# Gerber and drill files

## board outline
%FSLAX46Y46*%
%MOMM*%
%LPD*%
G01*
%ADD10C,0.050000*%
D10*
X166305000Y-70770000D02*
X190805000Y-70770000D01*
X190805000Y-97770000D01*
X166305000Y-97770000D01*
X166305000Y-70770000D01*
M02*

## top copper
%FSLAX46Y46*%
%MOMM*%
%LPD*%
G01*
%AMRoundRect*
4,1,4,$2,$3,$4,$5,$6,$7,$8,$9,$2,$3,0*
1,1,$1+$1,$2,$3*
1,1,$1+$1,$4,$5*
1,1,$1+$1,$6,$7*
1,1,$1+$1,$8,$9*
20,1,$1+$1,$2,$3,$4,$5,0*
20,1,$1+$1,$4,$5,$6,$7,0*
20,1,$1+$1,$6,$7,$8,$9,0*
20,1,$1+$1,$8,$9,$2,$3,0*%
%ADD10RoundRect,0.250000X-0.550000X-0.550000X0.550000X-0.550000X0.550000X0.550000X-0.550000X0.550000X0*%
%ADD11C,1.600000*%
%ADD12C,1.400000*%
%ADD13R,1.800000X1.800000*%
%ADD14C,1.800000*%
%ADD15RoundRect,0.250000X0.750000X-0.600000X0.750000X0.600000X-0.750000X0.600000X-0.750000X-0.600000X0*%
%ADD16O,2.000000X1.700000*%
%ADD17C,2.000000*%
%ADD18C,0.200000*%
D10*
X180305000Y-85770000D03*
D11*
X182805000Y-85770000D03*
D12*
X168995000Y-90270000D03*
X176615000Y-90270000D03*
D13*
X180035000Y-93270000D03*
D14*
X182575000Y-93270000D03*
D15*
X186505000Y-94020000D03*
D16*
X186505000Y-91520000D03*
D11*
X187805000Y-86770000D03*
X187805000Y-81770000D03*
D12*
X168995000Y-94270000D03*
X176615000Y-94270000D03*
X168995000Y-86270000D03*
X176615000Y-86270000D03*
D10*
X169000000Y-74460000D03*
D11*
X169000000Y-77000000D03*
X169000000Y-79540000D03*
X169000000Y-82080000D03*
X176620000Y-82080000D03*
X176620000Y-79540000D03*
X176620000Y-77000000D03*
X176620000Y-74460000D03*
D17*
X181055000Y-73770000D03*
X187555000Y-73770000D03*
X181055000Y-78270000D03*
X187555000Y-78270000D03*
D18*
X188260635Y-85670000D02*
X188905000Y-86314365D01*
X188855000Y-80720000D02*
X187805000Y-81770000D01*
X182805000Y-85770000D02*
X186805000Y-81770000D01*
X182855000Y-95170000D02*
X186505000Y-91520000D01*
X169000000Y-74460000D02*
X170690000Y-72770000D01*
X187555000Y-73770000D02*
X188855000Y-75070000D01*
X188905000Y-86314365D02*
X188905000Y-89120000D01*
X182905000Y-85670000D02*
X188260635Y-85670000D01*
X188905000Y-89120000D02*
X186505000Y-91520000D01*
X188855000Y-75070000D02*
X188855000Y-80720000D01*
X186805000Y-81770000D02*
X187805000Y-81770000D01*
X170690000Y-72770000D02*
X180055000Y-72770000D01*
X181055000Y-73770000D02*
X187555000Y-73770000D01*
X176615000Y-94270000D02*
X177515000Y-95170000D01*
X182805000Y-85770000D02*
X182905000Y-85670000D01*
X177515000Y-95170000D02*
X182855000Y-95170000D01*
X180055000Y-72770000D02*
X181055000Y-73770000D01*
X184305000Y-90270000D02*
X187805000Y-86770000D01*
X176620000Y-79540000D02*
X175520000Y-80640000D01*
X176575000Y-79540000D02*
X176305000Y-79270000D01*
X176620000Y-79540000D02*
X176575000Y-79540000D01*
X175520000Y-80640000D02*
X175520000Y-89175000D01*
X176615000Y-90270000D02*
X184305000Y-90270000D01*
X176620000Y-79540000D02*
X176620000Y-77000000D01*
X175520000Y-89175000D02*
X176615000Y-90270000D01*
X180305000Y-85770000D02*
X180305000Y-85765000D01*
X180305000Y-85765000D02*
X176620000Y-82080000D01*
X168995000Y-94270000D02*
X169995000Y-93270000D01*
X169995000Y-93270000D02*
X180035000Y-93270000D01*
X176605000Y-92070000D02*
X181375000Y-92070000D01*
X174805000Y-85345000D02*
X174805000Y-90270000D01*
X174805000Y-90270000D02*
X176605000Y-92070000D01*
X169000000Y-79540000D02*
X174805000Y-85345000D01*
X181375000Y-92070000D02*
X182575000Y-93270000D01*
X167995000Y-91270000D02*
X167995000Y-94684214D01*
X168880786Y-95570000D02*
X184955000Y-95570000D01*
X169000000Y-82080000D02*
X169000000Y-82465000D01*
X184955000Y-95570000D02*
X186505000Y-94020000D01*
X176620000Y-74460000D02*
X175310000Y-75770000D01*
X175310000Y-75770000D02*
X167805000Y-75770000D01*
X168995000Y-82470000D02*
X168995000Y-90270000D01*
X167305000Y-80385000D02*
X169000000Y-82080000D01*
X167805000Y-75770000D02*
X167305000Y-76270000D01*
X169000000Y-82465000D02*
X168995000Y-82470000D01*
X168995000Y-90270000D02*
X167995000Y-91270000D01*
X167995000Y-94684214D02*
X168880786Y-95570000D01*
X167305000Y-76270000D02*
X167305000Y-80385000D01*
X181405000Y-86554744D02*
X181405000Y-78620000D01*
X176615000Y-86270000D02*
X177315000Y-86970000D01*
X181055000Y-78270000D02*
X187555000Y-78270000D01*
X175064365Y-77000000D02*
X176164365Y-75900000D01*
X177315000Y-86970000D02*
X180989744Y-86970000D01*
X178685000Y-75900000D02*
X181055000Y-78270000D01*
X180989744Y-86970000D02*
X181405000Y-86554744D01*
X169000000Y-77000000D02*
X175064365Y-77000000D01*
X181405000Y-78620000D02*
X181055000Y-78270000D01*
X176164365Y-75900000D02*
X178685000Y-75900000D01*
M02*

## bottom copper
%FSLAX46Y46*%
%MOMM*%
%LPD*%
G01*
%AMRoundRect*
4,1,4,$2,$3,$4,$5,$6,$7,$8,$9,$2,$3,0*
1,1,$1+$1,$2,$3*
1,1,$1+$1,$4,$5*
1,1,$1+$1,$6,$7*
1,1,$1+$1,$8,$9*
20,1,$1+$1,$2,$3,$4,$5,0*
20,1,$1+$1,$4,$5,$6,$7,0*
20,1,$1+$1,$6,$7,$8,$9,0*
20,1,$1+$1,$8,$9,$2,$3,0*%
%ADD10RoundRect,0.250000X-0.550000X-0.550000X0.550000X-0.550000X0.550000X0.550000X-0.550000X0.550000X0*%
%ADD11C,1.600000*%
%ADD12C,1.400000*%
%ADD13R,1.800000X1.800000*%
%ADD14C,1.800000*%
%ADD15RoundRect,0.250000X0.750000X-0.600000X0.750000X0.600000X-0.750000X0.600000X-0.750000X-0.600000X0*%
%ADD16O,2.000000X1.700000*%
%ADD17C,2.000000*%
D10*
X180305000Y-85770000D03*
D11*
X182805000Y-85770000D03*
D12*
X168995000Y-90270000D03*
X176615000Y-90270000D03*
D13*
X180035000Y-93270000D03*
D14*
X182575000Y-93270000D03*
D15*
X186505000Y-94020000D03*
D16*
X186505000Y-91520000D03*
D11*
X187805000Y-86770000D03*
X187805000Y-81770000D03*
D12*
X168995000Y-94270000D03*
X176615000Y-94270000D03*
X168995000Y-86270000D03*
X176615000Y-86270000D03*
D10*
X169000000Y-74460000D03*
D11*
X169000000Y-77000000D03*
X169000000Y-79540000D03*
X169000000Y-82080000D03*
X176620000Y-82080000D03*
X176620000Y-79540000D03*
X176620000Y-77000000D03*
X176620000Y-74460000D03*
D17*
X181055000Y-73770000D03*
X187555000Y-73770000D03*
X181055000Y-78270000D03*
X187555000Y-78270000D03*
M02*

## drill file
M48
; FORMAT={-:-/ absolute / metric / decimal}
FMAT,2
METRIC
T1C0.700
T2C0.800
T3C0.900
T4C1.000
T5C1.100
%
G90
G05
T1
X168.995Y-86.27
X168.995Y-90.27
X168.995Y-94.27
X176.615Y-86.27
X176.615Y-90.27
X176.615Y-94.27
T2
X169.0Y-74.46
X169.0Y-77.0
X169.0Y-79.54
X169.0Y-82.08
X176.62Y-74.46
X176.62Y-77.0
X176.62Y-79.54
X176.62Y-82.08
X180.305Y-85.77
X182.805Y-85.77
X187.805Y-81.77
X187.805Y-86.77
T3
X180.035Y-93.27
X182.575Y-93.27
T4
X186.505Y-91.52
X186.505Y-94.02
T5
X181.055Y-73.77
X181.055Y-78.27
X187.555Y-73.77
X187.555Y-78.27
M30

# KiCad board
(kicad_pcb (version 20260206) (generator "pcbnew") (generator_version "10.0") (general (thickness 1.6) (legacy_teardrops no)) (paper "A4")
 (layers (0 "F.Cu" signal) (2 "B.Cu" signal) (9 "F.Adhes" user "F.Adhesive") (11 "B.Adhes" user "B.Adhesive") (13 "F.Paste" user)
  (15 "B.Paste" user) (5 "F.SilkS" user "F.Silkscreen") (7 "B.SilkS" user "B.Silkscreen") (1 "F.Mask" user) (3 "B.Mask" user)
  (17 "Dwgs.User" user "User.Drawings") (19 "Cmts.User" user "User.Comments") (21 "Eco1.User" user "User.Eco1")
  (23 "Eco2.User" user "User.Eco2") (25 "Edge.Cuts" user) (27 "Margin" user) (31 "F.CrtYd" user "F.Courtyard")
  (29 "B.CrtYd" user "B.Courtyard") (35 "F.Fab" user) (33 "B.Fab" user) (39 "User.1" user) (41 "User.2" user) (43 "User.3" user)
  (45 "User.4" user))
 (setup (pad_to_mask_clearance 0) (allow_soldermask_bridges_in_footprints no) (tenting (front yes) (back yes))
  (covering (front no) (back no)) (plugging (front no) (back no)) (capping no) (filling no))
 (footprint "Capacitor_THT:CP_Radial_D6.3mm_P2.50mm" (layer "F.Cu") (at 180.305 85.77)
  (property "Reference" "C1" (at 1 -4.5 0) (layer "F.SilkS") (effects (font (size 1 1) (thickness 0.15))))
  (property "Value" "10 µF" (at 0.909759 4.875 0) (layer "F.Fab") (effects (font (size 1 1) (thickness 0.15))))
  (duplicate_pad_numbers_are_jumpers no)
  (pad "1" thru_hole roundrect (at 0 0) (size 1.6 1.6) (drill 0.8) (layers "*.Cu" "*.Mask") (remove_unused_layers no)
   (roundrect_rratio 0.15625) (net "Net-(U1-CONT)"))
  (pad "2" thru_hole circle (at 2.5 0) (size 1.6 1.6) (drill 0.8) (layers "*.Cu" "*.Mask") (remove_unused_layers no) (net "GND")))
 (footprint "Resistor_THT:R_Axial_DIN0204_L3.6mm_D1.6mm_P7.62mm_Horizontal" (layer "F.Cu") (at 168.995 90.27)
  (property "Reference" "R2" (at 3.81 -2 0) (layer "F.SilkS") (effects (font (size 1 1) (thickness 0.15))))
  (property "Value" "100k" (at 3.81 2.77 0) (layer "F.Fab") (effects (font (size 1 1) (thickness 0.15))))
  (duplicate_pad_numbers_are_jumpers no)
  (pad "1" thru_hole circle (at 0 0) (size 1.4 1.4) (drill 0.7) (layers "*.Cu" "*.Mask") (remove_unused_layers no) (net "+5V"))
  (pad "2" thru_hole circle (at 7.62 0) (size 1.4 1.4) (drill 0.7) (layers "*.Cu" "*.Mask") (remove_unused_layers no) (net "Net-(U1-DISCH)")))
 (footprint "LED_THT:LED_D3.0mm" (layer "F.Cu") (at 180.035 93.27)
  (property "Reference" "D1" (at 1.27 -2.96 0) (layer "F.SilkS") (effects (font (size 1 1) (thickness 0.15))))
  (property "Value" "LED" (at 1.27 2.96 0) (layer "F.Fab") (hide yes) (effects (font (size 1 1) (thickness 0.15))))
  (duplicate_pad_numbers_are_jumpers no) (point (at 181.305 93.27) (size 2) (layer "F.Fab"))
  (pad "1" thru_hole rect (at 0 0) (size 1.8 1.8) (drill 0.9) (layers "*.Cu" "*.Mask") (remove_unused_layers no) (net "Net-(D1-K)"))
  (pad "2" thru_hole circle (at 2.54 0) (size 1.8 1.8) (drill 0.9) (layers "*.Cu" "*.Mask") (remove_unused_layers no) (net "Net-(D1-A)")))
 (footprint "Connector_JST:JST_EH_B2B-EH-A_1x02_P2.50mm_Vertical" (layer "F.Cu") (at 186.505 94.02 90)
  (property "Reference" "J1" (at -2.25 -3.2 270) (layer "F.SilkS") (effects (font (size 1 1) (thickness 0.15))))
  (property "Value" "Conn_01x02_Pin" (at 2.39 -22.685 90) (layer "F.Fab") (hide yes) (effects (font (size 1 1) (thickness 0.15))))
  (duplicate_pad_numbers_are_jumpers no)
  (pad "1" thru_hole roundrect (at 0 0 90) (size 1.7 2) (drill 1) (layers "*.Cu" "*.Mask") (remove_unused_layers no)
   (roundrect_rratio 0.147059) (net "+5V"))
  (pad "2" thru_hole oval (at 2.5 0 90) (size 1.7 2) (drill 1) (layers "*.Cu" "*.Mask") (remove_unused_layers no) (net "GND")))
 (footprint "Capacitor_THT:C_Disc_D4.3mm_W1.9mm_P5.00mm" (layer "F.Cu") (at 187.805 86.77 90)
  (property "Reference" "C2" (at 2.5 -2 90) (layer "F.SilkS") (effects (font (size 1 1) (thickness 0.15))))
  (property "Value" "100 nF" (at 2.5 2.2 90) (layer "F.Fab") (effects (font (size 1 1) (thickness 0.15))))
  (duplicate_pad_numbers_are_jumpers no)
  (pad "1" thru_hole circle (at 0 0 90) (size 1.6 1.6) (drill 0.8) (layers "*.Cu" "*.Mask") (remove_unused_layers no) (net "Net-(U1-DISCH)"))
  (pad "2" thru_hole circle (at 5 0 90) (size 1.6 1.6) (drill 0.8) (layers "*.Cu" "*.Mask") (remove_unused_layers no) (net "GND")))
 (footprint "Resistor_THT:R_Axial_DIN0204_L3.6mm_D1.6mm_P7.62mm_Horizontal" (layer "F.Cu") (at 168.995 94.27)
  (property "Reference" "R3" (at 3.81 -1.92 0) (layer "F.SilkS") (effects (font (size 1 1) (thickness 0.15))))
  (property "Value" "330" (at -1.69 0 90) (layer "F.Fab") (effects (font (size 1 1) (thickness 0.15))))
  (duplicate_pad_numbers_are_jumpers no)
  (pad "1" thru_hole circle (at 0 0) (size 1.4 1.4) (drill 0.7) (layers "*.Cu" "*.Mask") (remove_unused_layers no) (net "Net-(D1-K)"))
  (pad "2" thru_hole circle (at 7.62 0) (size 1.4 1.4) (drill 0.7) (layers "*.Cu" "*.Mask") (remove_unused_layers no) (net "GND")))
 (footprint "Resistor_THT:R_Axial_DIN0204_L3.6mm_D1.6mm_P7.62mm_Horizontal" (layer "F.Cu") (at 168.995 86.27)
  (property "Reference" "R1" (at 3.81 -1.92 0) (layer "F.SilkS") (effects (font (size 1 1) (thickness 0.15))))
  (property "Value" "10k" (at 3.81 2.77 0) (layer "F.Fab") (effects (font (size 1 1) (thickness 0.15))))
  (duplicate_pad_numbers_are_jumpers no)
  (pad "1" thru_hole circle (at 0 0) (size 1.4 1.4) (drill 0.7) (layers "*.Cu" "*.Mask") (remove_unused_layers no) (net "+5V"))
  (pad "2" thru_hole circle (at 7.62 0) (size 1.4 1.4) (drill 0.7) (layers "*.Cu" "*.Mask") (remove_unused_layers no) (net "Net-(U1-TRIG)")))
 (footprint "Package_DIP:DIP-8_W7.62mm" (layer "F.Cu") (at 169 74.46)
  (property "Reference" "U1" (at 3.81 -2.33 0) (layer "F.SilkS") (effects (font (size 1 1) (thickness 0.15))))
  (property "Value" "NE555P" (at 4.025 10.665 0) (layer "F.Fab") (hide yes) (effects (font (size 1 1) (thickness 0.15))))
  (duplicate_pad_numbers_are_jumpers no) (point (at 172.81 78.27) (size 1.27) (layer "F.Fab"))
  (pad "1" thru_hole roundrect (at 0 0) (size 1.6 1.6) (drill 0.8) (layers "*.Cu" "*.Mask") (remove_unused_layers no)
   (roundrect_rratio 0.15625) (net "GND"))
  (pad "2" thru_hole circle (at 0 2.54) (size 1.6 1.6) (drill 0.8) (layers "*.Cu" "*.Mask") (remove_unused_layers no) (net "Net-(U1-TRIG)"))
  (pad "3" thru_hole circle (at 0 5.08) (size 1.6 1.6) (drill 0.8) (layers "*.Cu" "*.Mask") (remove_unused_layers no) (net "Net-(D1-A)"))
  (pad "4" thru_hole circle (at 0 7.62) (size 1.6 1.6) (drill 0.8) (layers "*.Cu" "*.Mask") (remove_unused_layers no) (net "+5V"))
  (pad "5" thru_hole circle (at 7.62 7.62) (size 1.6 1.6) (drill 0.8) (layers "*.Cu" "*.Mask") (remove_unused_layers no)
   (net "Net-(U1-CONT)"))
  (pad "6" thru_hole circle (at 7.62 5.08) (size 1.6 1.6) (drill 0.8) (layers "*.Cu" "*.Mask") (remove_unused_layers no)
   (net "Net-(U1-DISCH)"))
  (pad "7" thru_hole circle (at 7.62 2.54) (size 1.6 1.6) (drill 0.8) (layers "*.Cu" "*.Mask") (remove_unused_layers no)
   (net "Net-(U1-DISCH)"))
  (pad "8" thru_hole circle (at 7.62 0) (size 1.6 1.6) (drill 0.8) (layers "*.Cu" "*.Mask") (remove_unused_layers no) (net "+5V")))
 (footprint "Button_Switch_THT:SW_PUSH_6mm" (layer "F.Cu") (at 181.055 73.77)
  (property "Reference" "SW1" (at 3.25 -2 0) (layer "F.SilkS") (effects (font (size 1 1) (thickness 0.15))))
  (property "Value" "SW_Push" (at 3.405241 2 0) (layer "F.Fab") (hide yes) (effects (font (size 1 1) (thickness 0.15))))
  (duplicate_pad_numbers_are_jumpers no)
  (pad "1" thru_hole circle (at 0 0 90) (size 2 2) (drill 1.1) (layers "*.Cu" "*.Mask") (remove_unused_layers no) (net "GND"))
  (pad "1" thru_hole circle (at 6.5 0 90) (size 2 2) (drill 1.1) (layers "*.Cu" "*.Mask") (remove_unused_layers no) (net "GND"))
  (pad "2" thru_hole circle (at 0 4.5 90) (size 2 2) (drill 1.1) (layers "*.Cu" "*.Mask") (remove_unused_layers no) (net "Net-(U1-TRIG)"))
  (pad "2" thru_hole circle (at 6.5 4.5 90) (size 2 2) (drill 1.1) (layers "*.Cu" "*.Mask") (remove_unused_layers no) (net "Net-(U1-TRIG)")))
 (gr_rect (start 166.305 70.77) (end 190.805 97.77) (stroke (width 0.05) (type default)) (fill no) (layer "Edge.Cuts"))
 (segment (start 188.260635 85.67) (end 188.905 86.314365) (width 0.2) (layer "F.Cu") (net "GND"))
 (segment (start 188.855 80.72) (end 187.805 81.77) (width 0.2) (layer "F.Cu") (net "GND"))
 (segment (start 182.805 85.77) (end 186.805 81.77) (width 0.2) (layer "F.Cu") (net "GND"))
 (segment (start 182.855 95.17) (end 186.505 91.52) (width 0.2) (layer "F.Cu") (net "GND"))
 (segment (start 169 74.46) (end 170.69 72.77) (width 0.2) (layer "F.Cu") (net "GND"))
 (segment (start 187.555 73.77) (end 188.855 75.07) (width 0.2) (layer "F.Cu") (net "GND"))
 (segment (start 188.905 86.314365) (end 188.905 89.12) (width 0.2) (layer "F.Cu") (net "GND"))
 (segment (start 182.905 85.67) (end 188.260635 85.67) (width 0.2) (layer "F.Cu") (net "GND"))
 (segment (start 188.905 89.12) (end 186.505 91.52) (width 0.2) (layer "F.Cu") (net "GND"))
 (segment (start 188.855 75.07) (end 188.855 80.72) (width 0.2) (layer "F.Cu") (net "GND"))
 (segment (start 186.805 81.77) (end 187.805 81.77) (width 0.2) (layer "F.Cu") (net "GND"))
 (segment (start 170.69 72.77) (end 180.055 72.77) (width 0.2) (layer "F.Cu") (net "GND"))
 (segment (start 181.055 73.77) (end 187.555 73.77) (width 0.2) (layer "F.Cu") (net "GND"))
 (segment (start 176.615 94.27) (end 177.515 95.17) (width 0.2) (layer "F.Cu") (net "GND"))
 (segment (start 182.805 85.77) (end 182.905 85.67) (width 0.2) (layer "F.Cu") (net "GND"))
 (segment (start 177.515 95.17) (end 182.855 95.17) (width 0.2) (layer "F.Cu") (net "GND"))
 (segment (start 180.055 72.77) (end 181.055 73.77) (width 0.2) (layer "F.Cu") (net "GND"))
 (segment (start 184.305 90.27) (end 187.805 86.77) (width 0.2) (layer "F.Cu") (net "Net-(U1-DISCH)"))
 (segment (start 176.62 79.54) (end 175.52 80.64) (width 0.2) (layer "F.Cu") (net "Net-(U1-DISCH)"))
 (segment (start 176.575 79.54) (end 176.305 79.27) (width 0.2) (layer "F.Cu") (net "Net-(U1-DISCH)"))
 (segment (start 176.62 79.54) (end 176.575 79.54) (width 0.2) (layer "F.Cu") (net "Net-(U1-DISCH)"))
 (segment (start 175.52 80.64) (end 175.52 89.175) (width 0.2) (layer "F.Cu") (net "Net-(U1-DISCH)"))
 (segment (start 176.615 90.27) (end 184.305 90.27) (width 0.2) (layer "F.Cu") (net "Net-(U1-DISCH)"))
 (segment (start 176.62 79.54) (end 176.62 77) (width 0.2) (layer "F.Cu") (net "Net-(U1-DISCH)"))
 (segment (start 175.52 89.175) (end 176.615 90.27) (width 0.2) (layer "F.Cu") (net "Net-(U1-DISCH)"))
 (segment (start 180.305 85.77) (end 180.305 85.765) (width 0.2) (layer "F.Cu") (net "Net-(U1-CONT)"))
 (segment (start 180.305 85.765) (end 176.62 82.08) (width 0.2) (layer "F.Cu") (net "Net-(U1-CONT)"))
 (segment (start 168.995 94.27) (end 169.995 93.27) (width 0.2) (layer "F.Cu") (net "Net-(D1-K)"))
 (segment (start 169.995 93.27) (end 180.035 93.27) (width 0.2) (layer "F.Cu") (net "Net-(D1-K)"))
 (segment (start 176.605 92.07) (end 181.375 92.07) (width 0.2) (layer "F.Cu") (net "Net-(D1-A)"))
 (segment (start 174.805 85.345) (end 174.805 90.27) (width 0.2) (layer "F.Cu") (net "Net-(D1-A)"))
 (segment (start 174.805 90.27) (end 176.605 92.07) (width 0.2) (layer "F.Cu") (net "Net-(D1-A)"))
 (segment (start 169 79.54) (end 174.805 85.345) (width 0.2) (layer "F.Cu") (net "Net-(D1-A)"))
 (segment (start 181.375 92.07) (end 182.575 93.27) (width 0.2) (layer "F.Cu") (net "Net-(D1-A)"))
 (segment (start 167.995 91.27) (end 167.995 94.684214) (width 0.2) (layer "F.Cu") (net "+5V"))
 (segment (start 168.880786 95.57) (end 184.955 95.57) (width 0.2) (layer "F.Cu") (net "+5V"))
 (segment (start 169 82.08) (end 169 82.465) (width 0.2) (layer "F.Cu") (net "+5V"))
 (segment (start 184.955 95.57) (end 186.505 94.02) (width 0.2) (layer "F.Cu") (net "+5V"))
 (segment (start 176.62 74.46) (end 175.31 75.77) (width 0.2) (layer "F.Cu") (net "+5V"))
 (segment (start 175.31 75.77) (end 167.805 75.77) (width 0.2) (layer "F.Cu") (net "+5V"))
 (segment (start 168.995 82.47) (end 168.995 90.27) (width 0.2) (layer "F.Cu") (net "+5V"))
 (segment (start 167.305 80.385) (end 169 82.08) (width 0.2) (layer "F.Cu") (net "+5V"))
 (segment (start 167.805 75.77) (end 167.305 76.27) (width 0.2) (layer "F.Cu") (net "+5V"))
 (segment (start 169 82.465) (end 168.995 82.47) (width 0.2) (layer "F.Cu") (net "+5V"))
 (segment (start 168.995 90.27) (end 167.995 91.27) (width 0.2) (layer "F.Cu") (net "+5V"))
 (segment (start 167.995 94.684214) (end 168.880786 95.57) (width 0.2) (layer "F.Cu") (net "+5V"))
 (segment (start 167.305 76.27) (end 167.305 80.385) (width 0.2) (layer "F.Cu") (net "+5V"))
 (segment (start 181.405 86.554744) (end 181.405 78.62) (width 0.2) (layer "F.Cu") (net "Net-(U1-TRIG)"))
 (segment (start 176.615 86.27) (end 177.315 86.97) (width 0.2) (layer "F.Cu") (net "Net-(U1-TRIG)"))
 (segment (start 181.055 78.27) (end 187.555 78.27) (width 0.2) (layer "F.Cu") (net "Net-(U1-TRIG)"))
 (segment (start 175.064365 77) (end 176.164365 75.9) (width 0.2) (layer "F.Cu") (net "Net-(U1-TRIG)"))
 (segment (start 177.315 86.97) (end 180.989744 86.97) (width 0.2) (layer "F.Cu") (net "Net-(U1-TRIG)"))
 (segment (start 178.685 75.9) (end 181.055 78.27) (width 0.2) (layer "F.Cu") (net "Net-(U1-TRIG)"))
 (segment (start 180.989744 86.97) (end 181.405 86.554744) (width 0.2) (layer "F.Cu") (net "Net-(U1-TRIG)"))
 (segment (start 169 77) (end 175.064365 77) (width 0.2) (layer "F.Cu") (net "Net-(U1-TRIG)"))
 (segment (start 181.405 78.62) (end 181.055 78.27) (width 0.2) (layer "F.Cu") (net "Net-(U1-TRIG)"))
 (segment (start 176.164365 75.9) (end 178.685 75.9) (width 0.2) (layer "F.Cu") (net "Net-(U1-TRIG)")))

